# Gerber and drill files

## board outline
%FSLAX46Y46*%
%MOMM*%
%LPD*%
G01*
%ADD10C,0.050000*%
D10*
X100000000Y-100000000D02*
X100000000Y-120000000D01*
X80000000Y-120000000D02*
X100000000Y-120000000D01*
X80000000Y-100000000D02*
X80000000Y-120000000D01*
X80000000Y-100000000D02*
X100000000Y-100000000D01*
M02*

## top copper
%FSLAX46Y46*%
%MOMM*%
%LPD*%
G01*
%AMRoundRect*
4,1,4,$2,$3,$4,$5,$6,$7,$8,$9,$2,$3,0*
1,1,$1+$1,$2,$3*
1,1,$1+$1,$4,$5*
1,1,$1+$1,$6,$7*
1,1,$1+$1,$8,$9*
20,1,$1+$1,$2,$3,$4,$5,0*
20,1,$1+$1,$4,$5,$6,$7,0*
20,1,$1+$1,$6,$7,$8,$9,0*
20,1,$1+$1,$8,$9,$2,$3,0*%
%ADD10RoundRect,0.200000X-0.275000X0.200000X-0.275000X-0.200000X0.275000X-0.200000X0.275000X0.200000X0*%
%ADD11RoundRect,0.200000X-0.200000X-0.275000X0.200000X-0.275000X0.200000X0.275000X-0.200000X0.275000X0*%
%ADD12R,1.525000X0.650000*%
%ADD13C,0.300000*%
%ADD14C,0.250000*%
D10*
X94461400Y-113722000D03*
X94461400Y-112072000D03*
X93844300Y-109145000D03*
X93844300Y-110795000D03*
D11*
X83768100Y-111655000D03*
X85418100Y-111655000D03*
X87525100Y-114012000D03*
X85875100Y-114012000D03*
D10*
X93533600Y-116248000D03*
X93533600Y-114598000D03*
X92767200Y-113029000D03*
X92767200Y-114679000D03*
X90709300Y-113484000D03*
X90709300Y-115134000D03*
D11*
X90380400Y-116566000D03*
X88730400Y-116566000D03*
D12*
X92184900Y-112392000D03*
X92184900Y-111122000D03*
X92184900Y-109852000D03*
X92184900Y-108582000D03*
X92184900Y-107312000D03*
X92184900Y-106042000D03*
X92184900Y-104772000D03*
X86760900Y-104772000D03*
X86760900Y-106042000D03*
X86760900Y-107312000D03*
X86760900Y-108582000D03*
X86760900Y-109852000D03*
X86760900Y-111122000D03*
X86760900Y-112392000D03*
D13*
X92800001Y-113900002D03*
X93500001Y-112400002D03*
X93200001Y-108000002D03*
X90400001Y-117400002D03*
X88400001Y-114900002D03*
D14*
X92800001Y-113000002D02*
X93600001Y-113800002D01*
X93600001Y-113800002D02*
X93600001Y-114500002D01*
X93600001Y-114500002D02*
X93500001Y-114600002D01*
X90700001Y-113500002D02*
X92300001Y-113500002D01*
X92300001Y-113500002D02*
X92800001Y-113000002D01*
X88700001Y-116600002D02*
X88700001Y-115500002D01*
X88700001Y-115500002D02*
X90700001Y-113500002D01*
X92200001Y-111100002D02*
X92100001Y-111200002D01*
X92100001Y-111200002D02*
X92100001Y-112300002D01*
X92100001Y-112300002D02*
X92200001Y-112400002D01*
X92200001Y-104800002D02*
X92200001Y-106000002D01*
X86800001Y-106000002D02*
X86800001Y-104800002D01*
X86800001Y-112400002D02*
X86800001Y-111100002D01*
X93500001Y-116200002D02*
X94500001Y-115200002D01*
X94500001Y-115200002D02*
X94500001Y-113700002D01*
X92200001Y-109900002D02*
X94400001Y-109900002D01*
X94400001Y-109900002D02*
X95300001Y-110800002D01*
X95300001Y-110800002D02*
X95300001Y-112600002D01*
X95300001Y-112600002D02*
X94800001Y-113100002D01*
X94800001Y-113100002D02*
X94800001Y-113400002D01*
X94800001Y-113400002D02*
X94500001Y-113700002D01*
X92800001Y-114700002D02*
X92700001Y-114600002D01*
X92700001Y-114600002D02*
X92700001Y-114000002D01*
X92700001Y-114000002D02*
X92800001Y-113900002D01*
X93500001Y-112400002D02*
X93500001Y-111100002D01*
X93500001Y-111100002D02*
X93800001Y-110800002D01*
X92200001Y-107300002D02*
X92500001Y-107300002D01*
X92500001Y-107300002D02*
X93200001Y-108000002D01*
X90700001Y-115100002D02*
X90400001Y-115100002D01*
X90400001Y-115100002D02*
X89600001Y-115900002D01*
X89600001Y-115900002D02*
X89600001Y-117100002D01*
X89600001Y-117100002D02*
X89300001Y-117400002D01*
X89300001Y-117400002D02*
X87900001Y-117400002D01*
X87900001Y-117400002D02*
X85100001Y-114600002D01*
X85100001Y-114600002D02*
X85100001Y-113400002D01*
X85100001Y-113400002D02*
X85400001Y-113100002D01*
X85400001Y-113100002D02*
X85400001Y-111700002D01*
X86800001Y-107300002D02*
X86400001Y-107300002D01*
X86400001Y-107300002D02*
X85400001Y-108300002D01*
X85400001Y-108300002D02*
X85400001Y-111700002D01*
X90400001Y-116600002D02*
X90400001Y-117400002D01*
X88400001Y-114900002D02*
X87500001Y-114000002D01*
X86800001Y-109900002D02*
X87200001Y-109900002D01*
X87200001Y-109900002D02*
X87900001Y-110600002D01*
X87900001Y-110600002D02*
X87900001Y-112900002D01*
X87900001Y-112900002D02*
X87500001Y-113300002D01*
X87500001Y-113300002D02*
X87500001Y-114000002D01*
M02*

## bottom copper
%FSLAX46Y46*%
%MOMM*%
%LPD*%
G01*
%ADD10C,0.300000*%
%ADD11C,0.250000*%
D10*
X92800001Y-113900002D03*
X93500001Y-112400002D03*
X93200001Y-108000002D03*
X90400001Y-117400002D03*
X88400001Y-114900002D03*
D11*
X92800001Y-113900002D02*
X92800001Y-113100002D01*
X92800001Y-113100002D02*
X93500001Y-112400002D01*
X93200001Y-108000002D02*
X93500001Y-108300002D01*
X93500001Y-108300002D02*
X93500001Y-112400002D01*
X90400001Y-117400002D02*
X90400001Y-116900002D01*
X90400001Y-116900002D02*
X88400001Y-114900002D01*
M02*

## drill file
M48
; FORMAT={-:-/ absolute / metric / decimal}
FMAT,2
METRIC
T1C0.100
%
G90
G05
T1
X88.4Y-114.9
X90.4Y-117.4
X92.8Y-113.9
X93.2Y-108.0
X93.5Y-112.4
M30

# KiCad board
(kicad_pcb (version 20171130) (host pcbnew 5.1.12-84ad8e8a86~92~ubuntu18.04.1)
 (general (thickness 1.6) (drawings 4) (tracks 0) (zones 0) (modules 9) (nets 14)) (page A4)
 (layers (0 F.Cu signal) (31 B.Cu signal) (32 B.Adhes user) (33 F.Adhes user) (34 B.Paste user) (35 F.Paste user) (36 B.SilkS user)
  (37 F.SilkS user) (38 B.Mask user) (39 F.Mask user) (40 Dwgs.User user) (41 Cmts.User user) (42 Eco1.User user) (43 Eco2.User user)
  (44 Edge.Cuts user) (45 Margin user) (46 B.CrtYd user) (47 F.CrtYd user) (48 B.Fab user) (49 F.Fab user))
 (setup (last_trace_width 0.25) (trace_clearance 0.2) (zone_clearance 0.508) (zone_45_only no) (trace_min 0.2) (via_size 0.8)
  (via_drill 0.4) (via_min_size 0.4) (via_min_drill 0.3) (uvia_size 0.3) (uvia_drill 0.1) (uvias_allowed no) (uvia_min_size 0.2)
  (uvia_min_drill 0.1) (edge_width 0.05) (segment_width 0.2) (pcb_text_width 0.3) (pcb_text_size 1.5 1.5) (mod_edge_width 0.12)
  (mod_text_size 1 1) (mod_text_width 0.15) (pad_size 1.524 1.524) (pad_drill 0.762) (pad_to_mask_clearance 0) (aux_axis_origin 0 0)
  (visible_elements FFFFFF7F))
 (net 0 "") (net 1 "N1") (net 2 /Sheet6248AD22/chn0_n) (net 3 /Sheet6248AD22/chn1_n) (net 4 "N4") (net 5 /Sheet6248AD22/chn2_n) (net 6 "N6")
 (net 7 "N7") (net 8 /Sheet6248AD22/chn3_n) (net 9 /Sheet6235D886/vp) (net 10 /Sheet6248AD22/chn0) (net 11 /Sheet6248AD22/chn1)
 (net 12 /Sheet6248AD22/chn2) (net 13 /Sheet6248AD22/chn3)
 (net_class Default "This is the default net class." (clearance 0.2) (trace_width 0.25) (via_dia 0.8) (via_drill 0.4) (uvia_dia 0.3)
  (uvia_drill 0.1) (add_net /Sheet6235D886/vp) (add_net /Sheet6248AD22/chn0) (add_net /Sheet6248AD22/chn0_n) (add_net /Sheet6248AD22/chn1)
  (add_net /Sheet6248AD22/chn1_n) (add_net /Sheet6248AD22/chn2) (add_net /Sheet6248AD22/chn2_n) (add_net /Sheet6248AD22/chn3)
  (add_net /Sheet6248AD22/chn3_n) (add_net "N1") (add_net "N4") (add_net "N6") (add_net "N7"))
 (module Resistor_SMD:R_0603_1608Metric (layer F.Cu) (at 94.461400 112.897000 270.000000)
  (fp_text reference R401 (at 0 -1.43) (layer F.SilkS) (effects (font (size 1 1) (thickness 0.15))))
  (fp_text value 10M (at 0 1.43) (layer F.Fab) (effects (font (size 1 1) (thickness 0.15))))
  (pad 2 smd roundrect (at 0.825 0 270.000000) (size 0.8 0.95) (layers F.Cu F.Mask F.Paste) (roundrect_rratio 0.25) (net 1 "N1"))
  (pad 1 smd roundrect (at -0.825 0 270.000000) (size 0.8 0.95) (layers F.Cu F.Mask F.Paste) (roundrect_rratio 0.25)
   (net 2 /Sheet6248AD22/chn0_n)))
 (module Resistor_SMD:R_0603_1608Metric (layer F.Cu) (at 93.844300 109.970000 270.000000)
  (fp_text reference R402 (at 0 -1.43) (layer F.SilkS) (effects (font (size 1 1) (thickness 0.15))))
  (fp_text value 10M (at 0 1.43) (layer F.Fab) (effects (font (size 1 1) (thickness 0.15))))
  (pad 1 smd roundrect (at -0.825 0 270.000000) (size 0.8 0.95) (layers F.Cu F.Mask F.Paste) (roundrect_rratio 0.25)
   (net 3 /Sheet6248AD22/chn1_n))
  (pad 2 smd roundrect (at 0.825 0 270.000000) (size 0.8 0.95) (layers F.Cu F.Mask F.Paste) (roundrect_rratio 0.25) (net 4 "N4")))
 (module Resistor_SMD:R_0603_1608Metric (layer F.Cu) (at 84.593100 111.655000)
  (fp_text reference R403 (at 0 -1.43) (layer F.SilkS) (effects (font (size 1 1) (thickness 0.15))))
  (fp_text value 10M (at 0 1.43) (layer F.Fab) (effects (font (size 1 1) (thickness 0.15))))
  (pad 1 smd roundrect (at -0.825 0) (size 0.8 0.95) (layers F.Cu F.Mask F.Paste) (roundrect_rratio 0.25) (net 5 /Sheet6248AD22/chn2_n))
  (pad 2 smd roundrect (at 0.825 0) (size 0.8 0.95) (layers F.Cu F.Mask F.Paste) (roundrect_rratio 0.25) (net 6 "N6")))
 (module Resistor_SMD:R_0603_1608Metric (layer F.Cu) (at 86.700100 114.012000)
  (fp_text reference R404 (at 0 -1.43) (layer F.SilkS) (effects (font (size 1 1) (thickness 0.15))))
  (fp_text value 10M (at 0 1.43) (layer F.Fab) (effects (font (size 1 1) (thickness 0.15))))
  (pad 2 smd roundrect (at 0.825 0) (size 0.8 0.95) (layers F.Cu F.Mask F.Paste) (roundrect_rratio 0.25) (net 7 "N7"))
  (pad 1 smd roundrect (at -0.825 0) (size 0.8 0.95) (layers F.Cu F.Mask F.Paste) (roundrect_rratio 0.25) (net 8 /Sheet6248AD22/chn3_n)))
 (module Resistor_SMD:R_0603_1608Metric (layer F.Cu) (at 93.533600 115.423000 270.000000)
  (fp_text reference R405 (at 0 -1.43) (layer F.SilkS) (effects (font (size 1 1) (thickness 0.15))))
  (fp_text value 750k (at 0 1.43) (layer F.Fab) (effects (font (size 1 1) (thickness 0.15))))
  (pad 2 smd roundrect (at 0.825 0 270.000000) (size 0.8 0.95) (layers F.Cu F.Mask F.Paste) (roundrect_rratio 0.25) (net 1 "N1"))
  (pad 1 smd roundrect (at -0.825 0 270.000000) (size 0.8 0.95) (layers F.Cu F.Mask F.Paste) (roundrect_rratio 0.25)
   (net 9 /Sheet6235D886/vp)))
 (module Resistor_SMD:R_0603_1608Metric (layer F.Cu) (at 92.767200 113.854000 270.000000)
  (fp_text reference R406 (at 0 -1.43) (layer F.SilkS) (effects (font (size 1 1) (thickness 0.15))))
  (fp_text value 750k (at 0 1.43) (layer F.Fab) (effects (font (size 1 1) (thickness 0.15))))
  (pad 1 smd roundrect (at -0.825 0 270.000000) (size 0.8 0.95) (layers F.Cu F.Mask F.Paste) (roundrect_rratio 0.25)
   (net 9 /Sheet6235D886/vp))
  (pad 2 smd roundrect (at 0.825 0 270.000000) (size 0.8 0.95) (layers F.Cu F.Mask F.Paste) (roundrect_rratio 0.25) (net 4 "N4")))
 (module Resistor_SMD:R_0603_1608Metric (layer F.Cu) (at 90.709300 114.309000 270.000000)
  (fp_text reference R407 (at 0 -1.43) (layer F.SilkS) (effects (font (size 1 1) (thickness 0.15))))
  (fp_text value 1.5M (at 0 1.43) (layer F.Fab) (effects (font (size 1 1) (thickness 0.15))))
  (pad 1 smd roundrect (at -0.825 0 270.000000) (size 0.8 0.95) (layers F.Cu F.Mask F.Paste) (roundrect_rratio 0.25)
   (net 9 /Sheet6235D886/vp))
  (pad 2 smd roundrect (at 0.825 0 270.000000) (size 0.8 0.95) (layers F.Cu F.Mask F.Paste) (roundrect_rratio 0.25) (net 6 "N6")))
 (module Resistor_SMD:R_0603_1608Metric (layer F.Cu) (at 89.555400 116.566000)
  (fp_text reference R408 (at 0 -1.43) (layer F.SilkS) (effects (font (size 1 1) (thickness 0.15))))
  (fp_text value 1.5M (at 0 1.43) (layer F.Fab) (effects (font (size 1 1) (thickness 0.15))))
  (pad 2 smd roundrect (at 0.825 0) (size 0.8 0.95) (layers F.Cu F.Mask F.Paste) (roundrect_rratio 0.25) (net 7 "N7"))
  (pad 1 smd roundrect (at -0.825 0) (size 0.8 0.95) (layers F.Cu F.Mask F.Paste) (roundrect_rratio 0.25) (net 9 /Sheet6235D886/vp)))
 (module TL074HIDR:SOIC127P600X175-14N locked (layer F.Cu) (at 89.472900 108.582000 180.000000)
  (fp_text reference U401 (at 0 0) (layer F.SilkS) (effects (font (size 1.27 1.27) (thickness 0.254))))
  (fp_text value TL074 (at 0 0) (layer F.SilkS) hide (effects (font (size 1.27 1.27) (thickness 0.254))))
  (pad 1 smd rect (at -2.712 -3.81 270.000000) (size 0.65 1.525) (layers F.Cu F.Mask F.Paste) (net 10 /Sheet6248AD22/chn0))
  (pad 2 smd rect (at -2.712 -2.54 270.000000) (size 0.65 1.525) (layers F.Cu F.Mask F.Paste) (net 10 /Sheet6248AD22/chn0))
  (pad 3 smd rect (at -2.712 -1.27 270.000000) (size 0.65 1.525) (layers F.Cu F.Mask F.Paste) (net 1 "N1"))
  (pad 4 smd rect (at -2.712 0 270.000000) (size 0.65 1.525) (layers F.Cu F.Mask F.Paste))
  (pad 5 smd rect (at -2.712 1.27 270.000000) (size 0.65 1.525) (layers F.Cu F.Mask F.Paste) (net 4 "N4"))
  (pad 6 smd rect (at -2.712 2.54 270.000000) (size 0.65 1.525) (layers F.Cu F.Mask F.Paste) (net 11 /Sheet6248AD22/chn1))
  (pad 7 smd rect (at -2.712 3.81 270.000000) (size 0.65 1.525) (layers F.Cu F.Mask F.Paste) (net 11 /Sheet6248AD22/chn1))
  (pad 8 smd rect (at 2.712 3.81 270.000000) (size 0.65 1.525) (layers F.Cu F.Mask F.Paste) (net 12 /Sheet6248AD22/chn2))
  (pad 9 smd rect (at 2.712 2.54 270.000000) (size 0.65 1.525) (layers F.Cu F.Mask F.Paste) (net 12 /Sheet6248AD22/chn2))
  (pad 10 smd rect (at 2.712 1.27 270.000000) (size 0.65 1.525) (layers F.Cu F.Mask F.Paste) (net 6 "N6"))
  (pad 11 smd rect (at 2.712 0 270.000000) (size 0.65 1.525) (layers F.Cu F.Mask F.Paste))
  (pad 12 smd rect (at 2.712 -1.27 270.000000) (size 0.65 1.525) (layers F.Cu F.Mask F.Paste) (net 7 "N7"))
  (pad 13 smd rect (at 2.712 -2.54 270.000000) (size 0.65 1.525) (layers F.Cu F.Mask F.Paste) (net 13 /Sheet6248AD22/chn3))
  (pad 14 smd rect (at 2.712 -3.81 270.000000) (size 0.65 1.525) (layers F.Cu F.Mask F.Paste) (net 13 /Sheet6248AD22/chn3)))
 (gr_line (start 100 100) (end 100 120) (layer Edge.Cuts) (width 0.05))
 (gr_line (start 80 120) (end 100 120) (layer Edge.Cuts) (width 0.05))
 (gr_line (start 80 100) (end 80 120) (layer Edge.Cuts) (width 0.05))
 (gr_line (start 80 100) (end 100 100) (layer Edge.Cuts) (width 0.05))
 (segment (start 92.800001 113.000002) (end 93.600001 113.800002) (width 0.250000) (layer F.Cu) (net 9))
 (segment (start 93.600001 113.800002) (end 93.600001 114.500002) (width 0.250000) (layer F.Cu) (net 9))
 (segment (start 93.600001 114.500002) (end 93.500001 114.600002) (width 0.250000) (layer F.Cu) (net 9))
 (segment (start 90.700001 113.500002) (end 92.300001 113.500002) (width 0.250000) (layer F.Cu) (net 9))
 (segment (start 92.300001 113.500002) (end 92.800001 113.000002) (width 0.250000) (layer F.Cu) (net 9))
 (segment (start 88.700001 116.600002) (end 88.700001 115.500002) (width 0.250000) (layer F.Cu) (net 9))
 (segment (start 88.700001 115.500002) (end 90.700001 113.500002) (width 0.250000) (layer F.Cu) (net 9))
 (segment (start 92.200001 111.100002) (end 92.100001 111.200002) (width 0.250000) (layer F.Cu) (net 10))
 (segment (start 92.100001 111.200002) (end 92.100001 112.300002) (width 0.250000) (layer F.Cu) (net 10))
 (segment (start 92.100001 112.300002) (end 92.200001 112.400002) (width 0.250000) (layer F.Cu) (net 10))
 (segment (start 92.200001 104.800002) (end 92.200001 106.000002) (width 0.250000) (layer F.Cu) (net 11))
 (segment (start 86.800001 106.000002) (end 86.800001 104.800002) (width 0.250000) (layer F.Cu) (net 12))
 (segment (start 86.800001 112.400002) (end 86.800001 111.100002) (width 0.250000) (layer F.Cu) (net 13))
 (segment (start 93.500001 116.200002) (end 94.500001 115.200002) (width 0.250000) (layer F.Cu) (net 1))
 (segment (start 94.500001 115.200002) (end 94.500001 113.700002) (width 0.250000) (layer F.Cu) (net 1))
 (segment (start 92.200001 109.900002) (end 94.400001 109.900002) (width 0.250000) (layer F.Cu) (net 1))
 (segment (start 94.400001 109.900002) (end 95.300001 110.800002) (width 0.250000) (layer F.Cu) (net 1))
 (segment (start 95.300001 110.800002) (end 95.300001 112.600002) (width 0.250000) (layer F.Cu) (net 1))
 (segment (start 95.300001 112.600002) (end 94.800001 113.100002) (width 0.250000) (layer F.Cu) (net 1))
 (segment (start 94.800001 113.100002) (end 94.800001 113.400002) (width 0.250000) (layer F.Cu) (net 1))
 (segment (start 94.800001 113.400002) (end 94.500001 113.700002) (width 0.250000) (layer F.Cu) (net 1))
 (segment (start 92.800001 114.700002) (end 92.700001 114.600002) (width 0.250000) (layer F.Cu) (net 4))
 (segment (start 92.700001 114.600002) (end 92.700001 114.000002) (width 0.250000) (layer F.Cu) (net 4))
 (segment (start 92.700001 114.000002) (end 92.800001 113.900002) (width 0.250000) (layer F.Cu) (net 4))
 (segment (start 92.800001 113.900002) (end 92.800001 113.100002) (width 0.250000) (layer B.Cu) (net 4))
 (segment (start 92.800001 113.100002) (end 93.500001 112.400002) (width 0.250000) (layer B.Cu) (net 4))
 (segment (start 93.500001 112.400002) (end 93.500001 111.100002) (width 0.250000) (layer F.Cu) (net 4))
 (segment (start 93.500001 111.100002) (end 93.800001 110.800002) (width 0.250000) (layer F.Cu) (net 4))
 (segment (start 92.200001 107.300002) (end 92.500001 107.300002) (width 0.250000) (layer F.Cu) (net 4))
 (segment (start 92.500001 107.300002) (end 93.200001 108.000002) (width 0.250000) (layer F.Cu) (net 4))
 (segment (start 93.200001 108.000002) (end 93.500001 108.300002) (width 0.250000) (layer B.Cu) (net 4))
 (segment (start 93.500001 108.300002) (end 93.500001 112.400002) (width 0.250000) (layer B.Cu) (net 4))
 (via micro (at 92.800001 113.900002) (size 0.300000) (drill 0.100000) (layers F.Cu B.Cu) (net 4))
 (via micro (at 93.500001 112.400002) (size 0.300000) (drill 0.100000) (layers F.Cu B.Cu) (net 4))
 (via micro (at 93.200001 108.000002) (size 0.300000) (drill 0.100000) (layers F.Cu B.Cu) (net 4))
 (segment (start 90.700001 115.100002) (end 90.400001 115.100002) (width 0.250000) (layer F.Cu) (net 6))
 (segment (start 90.400001 115.100002) (end 89.600001 115.900002) (width 0.250000) (layer F.Cu) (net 6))
 (segment (start 89.600001 115.900002) (end 89.600001 117.100002) (width 0.250000) (layer F.Cu) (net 6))
 (segment (start 89.600001 117.100002) (end 89.300001 117.400002) (width 0.250000) (layer F.Cu) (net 6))
 (segment (start 89.300001 117.400002) (end 87.900001 117.400002) (width 0.250000) (layer F.Cu) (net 6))
 (segment (start 87.900001 117.400002) (end 85.100001 114.600002) (width 0.250000) (layer F.Cu) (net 6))
 (segment (start 85.100001 114.600002) (end 85.100001 113.400002) (width 0.250000) (layer F.Cu) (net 6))
 (segment (start 85.100001 113.400002) (end 85.400001 113.100002) (width 0.250000) (layer F.Cu) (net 6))
 (segment (start 85.400001 113.100002) (end 85.400001 111.700002) (width 0.250000) (layer F.Cu) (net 6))
 (segment (start 86.800001 107.300002) (end 86.400001 107.300002) (width 0.250000) (layer F.Cu) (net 6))
 (segment (start 86.400001 107.300002) (end 85.400001 108.300002) (width 0.250000) (layer F.Cu) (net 6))
 (segment (start 85.400001 108.300002) (end 85.400001 111.700002) (width 0.250000) (layer F.Cu) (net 6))
 (segment (start 90.400001 116.600002) (end 90.400001 117.400002) (width 0.250000) (layer F.Cu) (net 7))
 (segment (start 90.400001 117.400002) (end 90.400001 116.900002) (width 0.250000) (layer B.Cu) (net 7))
 (segment (start 90.400001 116.900002) (end 88.400001 114.900002) (width 0.250000) (layer B.Cu) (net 7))
 (segment (start 88.400001 114.900002) (end 87.500001 114.000002) (width 0.250000) (layer F.Cu) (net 7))
 (segment (start 86.800001 109.900002) (end 87.200001 109.900002) (width 0.250000) (layer F.Cu) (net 7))
 (segment (start 87.200001 109.900002) (end 87.900001 110.600002) (width 0.250000) (layer F.Cu) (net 7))
 (segment (start 87.900001 110.600002) (end 87.900001 112.900002) (width 0.250000) (layer F.Cu) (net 7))
 (segment (start 87.900001 112.900002) (end 87.500001 113.300002) (width 0.250000) (layer F.Cu) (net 7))
 (segment (start 87.500001 113.300002) (end 87.500001 114.000002) (width 0.250000) (layer F.Cu) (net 7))
 (via micro (at 90.400001 117.400002) (size 0.300000) (drill 0.100000) (layers F.Cu B.Cu) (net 7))
 (via micro (at 88.400001 114.900002) (size 0.300000) (drill 0.100000) (layers F.Cu B.Cu) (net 7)))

